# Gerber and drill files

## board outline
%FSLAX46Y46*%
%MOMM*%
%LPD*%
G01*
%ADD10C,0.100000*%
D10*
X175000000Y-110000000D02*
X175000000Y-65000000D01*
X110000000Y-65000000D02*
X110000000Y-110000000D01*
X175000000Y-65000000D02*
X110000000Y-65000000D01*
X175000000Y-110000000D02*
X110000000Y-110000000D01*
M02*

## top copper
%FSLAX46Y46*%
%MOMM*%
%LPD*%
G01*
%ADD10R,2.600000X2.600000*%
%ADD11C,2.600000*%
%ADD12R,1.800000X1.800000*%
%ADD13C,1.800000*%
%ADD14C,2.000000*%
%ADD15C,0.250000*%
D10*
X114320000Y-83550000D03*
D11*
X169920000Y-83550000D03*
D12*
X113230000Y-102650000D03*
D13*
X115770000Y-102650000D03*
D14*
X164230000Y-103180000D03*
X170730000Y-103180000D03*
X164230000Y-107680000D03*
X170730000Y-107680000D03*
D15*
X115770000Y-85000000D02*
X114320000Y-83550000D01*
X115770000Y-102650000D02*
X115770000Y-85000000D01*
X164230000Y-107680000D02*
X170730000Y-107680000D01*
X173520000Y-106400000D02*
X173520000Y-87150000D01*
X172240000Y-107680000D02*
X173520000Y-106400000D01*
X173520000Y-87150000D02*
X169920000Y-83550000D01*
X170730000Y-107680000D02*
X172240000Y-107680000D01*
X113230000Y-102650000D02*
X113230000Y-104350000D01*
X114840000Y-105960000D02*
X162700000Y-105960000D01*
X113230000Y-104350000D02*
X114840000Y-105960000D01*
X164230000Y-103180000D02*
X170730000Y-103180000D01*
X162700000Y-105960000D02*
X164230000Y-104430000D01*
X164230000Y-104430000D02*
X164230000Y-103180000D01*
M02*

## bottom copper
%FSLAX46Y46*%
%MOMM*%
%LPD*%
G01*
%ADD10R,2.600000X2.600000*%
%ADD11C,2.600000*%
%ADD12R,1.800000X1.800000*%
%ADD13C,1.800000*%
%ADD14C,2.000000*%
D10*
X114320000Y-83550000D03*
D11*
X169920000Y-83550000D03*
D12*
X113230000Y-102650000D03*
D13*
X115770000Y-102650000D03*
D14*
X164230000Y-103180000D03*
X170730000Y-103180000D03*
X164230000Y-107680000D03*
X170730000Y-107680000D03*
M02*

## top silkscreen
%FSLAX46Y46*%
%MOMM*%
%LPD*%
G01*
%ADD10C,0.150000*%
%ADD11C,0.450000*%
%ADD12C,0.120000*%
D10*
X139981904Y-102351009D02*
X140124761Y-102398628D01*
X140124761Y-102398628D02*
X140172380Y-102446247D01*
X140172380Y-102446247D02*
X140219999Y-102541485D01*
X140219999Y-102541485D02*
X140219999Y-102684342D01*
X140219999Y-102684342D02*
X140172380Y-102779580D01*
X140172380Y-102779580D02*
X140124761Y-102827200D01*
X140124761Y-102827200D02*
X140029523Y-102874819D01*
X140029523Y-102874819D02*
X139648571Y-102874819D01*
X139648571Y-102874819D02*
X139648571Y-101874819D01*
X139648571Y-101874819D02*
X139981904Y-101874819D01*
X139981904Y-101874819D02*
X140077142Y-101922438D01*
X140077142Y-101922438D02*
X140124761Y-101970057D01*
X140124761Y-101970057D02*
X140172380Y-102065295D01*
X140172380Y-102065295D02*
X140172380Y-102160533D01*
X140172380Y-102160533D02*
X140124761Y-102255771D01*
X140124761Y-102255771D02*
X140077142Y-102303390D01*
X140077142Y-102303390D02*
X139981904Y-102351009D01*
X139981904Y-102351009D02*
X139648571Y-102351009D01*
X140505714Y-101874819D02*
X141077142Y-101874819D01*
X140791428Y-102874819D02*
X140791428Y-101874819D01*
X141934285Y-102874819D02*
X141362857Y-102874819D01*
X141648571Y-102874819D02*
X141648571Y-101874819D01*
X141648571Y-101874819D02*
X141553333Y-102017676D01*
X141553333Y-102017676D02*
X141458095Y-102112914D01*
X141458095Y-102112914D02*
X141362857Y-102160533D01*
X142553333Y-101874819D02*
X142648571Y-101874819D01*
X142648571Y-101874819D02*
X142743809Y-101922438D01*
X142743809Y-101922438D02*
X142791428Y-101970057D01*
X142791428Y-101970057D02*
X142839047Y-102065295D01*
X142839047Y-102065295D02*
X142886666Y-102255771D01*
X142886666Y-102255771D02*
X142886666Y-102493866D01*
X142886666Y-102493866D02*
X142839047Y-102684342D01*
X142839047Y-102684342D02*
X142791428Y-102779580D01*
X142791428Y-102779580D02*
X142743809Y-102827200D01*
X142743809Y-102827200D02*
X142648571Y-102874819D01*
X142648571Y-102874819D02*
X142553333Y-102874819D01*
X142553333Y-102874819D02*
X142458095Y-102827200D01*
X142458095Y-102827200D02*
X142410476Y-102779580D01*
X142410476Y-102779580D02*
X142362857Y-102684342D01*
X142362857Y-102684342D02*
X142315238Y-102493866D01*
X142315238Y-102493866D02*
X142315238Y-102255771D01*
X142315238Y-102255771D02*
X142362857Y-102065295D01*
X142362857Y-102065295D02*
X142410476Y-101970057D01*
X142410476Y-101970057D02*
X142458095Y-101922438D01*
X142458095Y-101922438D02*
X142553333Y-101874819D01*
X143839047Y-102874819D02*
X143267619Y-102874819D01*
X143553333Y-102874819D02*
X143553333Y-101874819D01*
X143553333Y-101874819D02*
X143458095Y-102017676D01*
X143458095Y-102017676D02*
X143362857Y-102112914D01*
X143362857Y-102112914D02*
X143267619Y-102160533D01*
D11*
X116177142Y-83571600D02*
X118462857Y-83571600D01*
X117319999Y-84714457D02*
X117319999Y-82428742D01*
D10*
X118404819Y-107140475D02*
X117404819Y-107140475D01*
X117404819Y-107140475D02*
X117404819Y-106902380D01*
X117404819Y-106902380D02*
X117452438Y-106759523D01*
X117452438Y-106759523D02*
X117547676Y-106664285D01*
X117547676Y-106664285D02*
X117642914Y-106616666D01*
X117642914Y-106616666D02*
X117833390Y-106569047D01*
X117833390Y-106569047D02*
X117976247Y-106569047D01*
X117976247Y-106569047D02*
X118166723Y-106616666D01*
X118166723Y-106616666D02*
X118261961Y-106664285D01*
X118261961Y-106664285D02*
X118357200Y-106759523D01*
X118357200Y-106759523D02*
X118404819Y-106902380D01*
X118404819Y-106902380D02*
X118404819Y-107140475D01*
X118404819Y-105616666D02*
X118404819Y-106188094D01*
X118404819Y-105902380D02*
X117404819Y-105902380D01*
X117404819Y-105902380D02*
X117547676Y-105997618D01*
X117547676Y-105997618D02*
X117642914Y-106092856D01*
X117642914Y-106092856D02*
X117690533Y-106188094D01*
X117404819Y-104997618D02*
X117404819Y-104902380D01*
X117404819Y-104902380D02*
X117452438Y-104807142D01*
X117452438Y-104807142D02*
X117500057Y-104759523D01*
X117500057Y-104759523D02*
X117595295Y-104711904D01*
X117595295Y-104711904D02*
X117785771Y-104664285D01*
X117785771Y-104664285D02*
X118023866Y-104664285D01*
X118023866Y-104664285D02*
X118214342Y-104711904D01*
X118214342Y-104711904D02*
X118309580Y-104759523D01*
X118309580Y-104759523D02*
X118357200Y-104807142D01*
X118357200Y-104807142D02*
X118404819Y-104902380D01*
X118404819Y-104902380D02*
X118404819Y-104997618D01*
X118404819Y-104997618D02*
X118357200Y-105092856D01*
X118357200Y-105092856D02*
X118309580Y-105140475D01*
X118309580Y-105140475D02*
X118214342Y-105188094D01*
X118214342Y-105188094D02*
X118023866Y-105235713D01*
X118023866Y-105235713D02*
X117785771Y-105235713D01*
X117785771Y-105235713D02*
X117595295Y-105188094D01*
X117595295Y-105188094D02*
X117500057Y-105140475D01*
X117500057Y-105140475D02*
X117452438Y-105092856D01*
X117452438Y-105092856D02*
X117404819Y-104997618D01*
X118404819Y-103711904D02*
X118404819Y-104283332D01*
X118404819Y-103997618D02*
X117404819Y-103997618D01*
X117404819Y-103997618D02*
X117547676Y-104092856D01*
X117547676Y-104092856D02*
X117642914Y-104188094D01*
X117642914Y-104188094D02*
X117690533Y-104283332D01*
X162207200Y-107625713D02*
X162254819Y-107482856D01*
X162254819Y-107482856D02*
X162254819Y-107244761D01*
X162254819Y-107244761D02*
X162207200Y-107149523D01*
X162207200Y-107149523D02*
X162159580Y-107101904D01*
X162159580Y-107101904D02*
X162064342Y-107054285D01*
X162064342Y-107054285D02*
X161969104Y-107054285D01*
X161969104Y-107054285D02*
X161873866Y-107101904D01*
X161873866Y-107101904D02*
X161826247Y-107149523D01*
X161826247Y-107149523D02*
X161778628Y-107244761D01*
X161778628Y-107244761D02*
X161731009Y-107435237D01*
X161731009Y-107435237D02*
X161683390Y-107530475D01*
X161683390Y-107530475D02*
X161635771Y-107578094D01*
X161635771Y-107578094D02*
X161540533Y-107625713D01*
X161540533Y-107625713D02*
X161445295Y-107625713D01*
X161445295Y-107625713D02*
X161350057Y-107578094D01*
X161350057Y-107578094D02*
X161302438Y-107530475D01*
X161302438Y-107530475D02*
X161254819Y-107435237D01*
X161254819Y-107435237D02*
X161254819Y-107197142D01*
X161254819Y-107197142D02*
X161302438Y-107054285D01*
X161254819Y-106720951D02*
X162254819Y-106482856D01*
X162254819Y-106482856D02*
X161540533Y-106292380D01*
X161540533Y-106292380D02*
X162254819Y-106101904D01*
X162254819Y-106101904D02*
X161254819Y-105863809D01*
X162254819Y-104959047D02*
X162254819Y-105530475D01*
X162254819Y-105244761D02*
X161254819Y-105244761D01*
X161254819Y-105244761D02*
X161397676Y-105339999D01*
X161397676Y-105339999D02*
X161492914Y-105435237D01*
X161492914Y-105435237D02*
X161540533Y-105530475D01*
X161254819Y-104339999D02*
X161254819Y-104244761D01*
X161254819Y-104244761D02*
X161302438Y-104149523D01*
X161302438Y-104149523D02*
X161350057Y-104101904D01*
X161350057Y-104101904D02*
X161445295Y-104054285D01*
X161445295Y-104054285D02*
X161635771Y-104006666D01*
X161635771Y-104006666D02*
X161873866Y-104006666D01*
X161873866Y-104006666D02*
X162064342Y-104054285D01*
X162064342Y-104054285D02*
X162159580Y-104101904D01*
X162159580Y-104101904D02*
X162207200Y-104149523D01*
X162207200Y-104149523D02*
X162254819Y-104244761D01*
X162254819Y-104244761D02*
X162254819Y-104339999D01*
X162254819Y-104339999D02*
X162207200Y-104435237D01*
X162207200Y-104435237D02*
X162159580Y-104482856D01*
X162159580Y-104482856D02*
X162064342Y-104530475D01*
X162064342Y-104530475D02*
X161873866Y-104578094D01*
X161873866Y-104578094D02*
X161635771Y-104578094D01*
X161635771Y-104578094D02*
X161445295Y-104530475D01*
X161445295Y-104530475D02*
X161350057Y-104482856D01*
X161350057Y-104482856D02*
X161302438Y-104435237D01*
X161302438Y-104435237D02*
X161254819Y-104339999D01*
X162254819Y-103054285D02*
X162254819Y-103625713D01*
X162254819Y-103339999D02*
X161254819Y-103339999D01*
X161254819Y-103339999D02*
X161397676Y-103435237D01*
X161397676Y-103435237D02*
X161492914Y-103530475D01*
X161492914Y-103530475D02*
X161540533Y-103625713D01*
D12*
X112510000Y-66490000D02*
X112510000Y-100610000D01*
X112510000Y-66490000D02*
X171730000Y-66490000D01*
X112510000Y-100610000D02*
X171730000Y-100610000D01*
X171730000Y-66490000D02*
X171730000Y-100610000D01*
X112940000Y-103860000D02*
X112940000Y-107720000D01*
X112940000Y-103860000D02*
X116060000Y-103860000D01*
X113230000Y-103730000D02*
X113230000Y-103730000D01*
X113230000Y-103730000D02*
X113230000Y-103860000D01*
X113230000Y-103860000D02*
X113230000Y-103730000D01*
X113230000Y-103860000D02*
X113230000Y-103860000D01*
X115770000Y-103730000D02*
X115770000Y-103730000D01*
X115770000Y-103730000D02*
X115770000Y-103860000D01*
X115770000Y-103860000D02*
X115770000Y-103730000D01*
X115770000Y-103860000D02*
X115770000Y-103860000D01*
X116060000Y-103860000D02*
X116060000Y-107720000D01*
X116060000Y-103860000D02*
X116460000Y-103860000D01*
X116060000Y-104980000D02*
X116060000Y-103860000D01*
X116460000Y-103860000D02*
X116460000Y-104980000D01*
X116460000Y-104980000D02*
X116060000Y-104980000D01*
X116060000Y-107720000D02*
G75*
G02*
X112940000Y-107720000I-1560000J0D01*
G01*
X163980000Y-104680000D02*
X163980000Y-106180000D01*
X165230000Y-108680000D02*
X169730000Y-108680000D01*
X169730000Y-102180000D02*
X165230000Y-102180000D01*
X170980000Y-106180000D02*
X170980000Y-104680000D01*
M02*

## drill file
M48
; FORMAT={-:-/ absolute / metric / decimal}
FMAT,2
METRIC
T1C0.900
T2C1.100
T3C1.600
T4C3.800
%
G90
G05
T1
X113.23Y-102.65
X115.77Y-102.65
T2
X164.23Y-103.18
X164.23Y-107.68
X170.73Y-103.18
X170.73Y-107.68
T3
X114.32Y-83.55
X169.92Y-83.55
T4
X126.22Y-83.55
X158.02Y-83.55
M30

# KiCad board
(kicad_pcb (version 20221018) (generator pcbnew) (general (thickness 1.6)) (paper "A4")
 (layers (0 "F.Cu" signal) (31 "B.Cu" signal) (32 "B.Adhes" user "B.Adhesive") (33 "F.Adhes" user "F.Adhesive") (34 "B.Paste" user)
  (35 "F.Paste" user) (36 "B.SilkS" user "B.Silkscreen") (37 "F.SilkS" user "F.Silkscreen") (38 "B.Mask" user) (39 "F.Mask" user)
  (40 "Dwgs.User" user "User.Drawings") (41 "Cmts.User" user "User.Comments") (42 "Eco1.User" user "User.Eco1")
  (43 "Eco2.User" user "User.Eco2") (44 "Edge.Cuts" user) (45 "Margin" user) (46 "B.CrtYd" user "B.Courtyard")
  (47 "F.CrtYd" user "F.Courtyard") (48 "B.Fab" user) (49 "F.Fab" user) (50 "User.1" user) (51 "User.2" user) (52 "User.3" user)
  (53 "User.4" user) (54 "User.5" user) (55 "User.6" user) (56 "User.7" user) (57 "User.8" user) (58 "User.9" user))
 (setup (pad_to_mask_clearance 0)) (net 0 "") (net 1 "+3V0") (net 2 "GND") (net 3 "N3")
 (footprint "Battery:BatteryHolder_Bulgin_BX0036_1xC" (layer "F.Cu") (at 114.32 83.55)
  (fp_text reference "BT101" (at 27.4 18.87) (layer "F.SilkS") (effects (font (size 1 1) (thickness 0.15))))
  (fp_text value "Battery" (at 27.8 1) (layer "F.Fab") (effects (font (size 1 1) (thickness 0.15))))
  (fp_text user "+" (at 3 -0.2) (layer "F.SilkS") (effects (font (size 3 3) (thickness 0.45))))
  (fp_line (start -1.81 -17.06) (end -1.81 17.06) (stroke (width 0.12) (type solid)) (layer "F.SilkS"))
  (fp_line (start -1.81 -17.06) (end 57.41 -17.06) (stroke (width 0.12) (type solid)) (layer "F.SilkS"))
  (fp_line (start -1.81 17.06) (end 57.41 17.06) (stroke (width 0.12) (type solid)) (layer "F.SilkS"))
  (fp_line (start 57.41 -17.06) (end 57.41 17.06) (stroke (width 0.12) (type solid)) (layer "F.SilkS"))
  (pad "" np_thru_hole circle (at 11.9 0) (size 3.8 3.8) (drill 3.8) (layers "*.Cu" "*.Mask"))
  (pad "" np_thru_hole circle (at 43.7 0) (size 3.8 3.8) (drill 3.8) (layers "*.Cu" "*.Mask"))
  (pad "1" thru_hole rect (at 0 0) (size 2.6 2.6) (drill 1.6) (layers "*.Cu" "*.Mask") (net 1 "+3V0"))
  (pad "2" thru_hole circle (at 55.6 0) (size 2.6 2.6) (drill 1.6) (layers "*.Cu" "*.Mask") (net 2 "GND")))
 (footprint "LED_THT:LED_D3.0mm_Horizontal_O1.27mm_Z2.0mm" (layer "F.Cu") (at 113.23 102.65)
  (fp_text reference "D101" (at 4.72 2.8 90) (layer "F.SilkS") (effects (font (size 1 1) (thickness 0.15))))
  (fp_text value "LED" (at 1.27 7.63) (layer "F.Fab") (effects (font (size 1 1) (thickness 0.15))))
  (fp_line (start -0.29 1.21) (end -0.29 5.07) (stroke (width 0.12) (type solid)) (layer "F.SilkS"))
  (fp_line (start -0.29 1.21) (end 2.83 1.21) (stroke (width 0.12) (type solid)) (layer "F.SilkS"))
  (fp_line (start 0 1.08) (end 0 1.08) (stroke (width 0.12) (type solid)) (layer "F.SilkS"))
  (fp_line (start 0 1.08) (end 0 1.21) (stroke (width 0.12) (type solid)) (layer "F.SilkS"))
  (fp_line (start 0 1.21) (end 0 1.08) (stroke (width 0.12) (type solid)) (layer "F.SilkS"))
  (fp_line (start 0 1.21) (end 0 1.21) (stroke (width 0.12) (type solid)) (layer "F.SilkS"))
  (fp_line (start 2.54 1.08) (end 2.54 1.08) (stroke (width 0.12) (type solid)) (layer "F.SilkS"))
  (fp_line (start 2.54 1.08) (end 2.54 1.21) (stroke (width 0.12) (type solid)) (layer "F.SilkS"))
  (fp_line (start 2.54 1.21) (end 2.54 1.08) (stroke (width 0.12) (type solid)) (layer "F.SilkS"))
  (fp_line (start 2.54 1.21) (end 2.54 1.21) (stroke (width 0.12) (type solid)) (layer "F.SilkS"))
  (fp_line (start 2.83 1.21) (end 2.83 5.07) (stroke (width 0.12) (type solid)) (layer "F.SilkS"))
  (fp_line (start 2.83 1.21) (end 3.23 1.21) (stroke (width 0.12) (type solid)) (layer "F.SilkS"))
  (fp_line (start 2.83 2.33) (end 2.83 1.21) (stroke (width 0.12) (type solid)) (layer "F.SilkS"))
  (fp_line (start 3.23 1.21) (end 3.23 2.33) (stroke (width 0.12) (type solid)) (layer "F.SilkS"))
  (fp_line (start 3.23 2.33) (end 2.83 2.33) (stroke (width 0.12) (type solid)) (layer "F.SilkS"))
  (fp_arc (start 2.83 5.07) (mid 1.27 6.63) (end -0.29 5.07) (stroke (width 0.12) (type solid)) (layer "F.SilkS"))
  (pad "1" thru_hole rect (at 0 0) (size 1.8 1.8) (drill 0.9) (layers "*.Cu" "*.Mask") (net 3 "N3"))
  (pad "2" thru_hole circle (at 2.54 0) (size 1.8 1.8) (drill 0.9) (layers "*.Cu" "*.Mask") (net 1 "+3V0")))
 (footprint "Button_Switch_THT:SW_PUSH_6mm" (layer "F.Cu") (at 164.23 103.18)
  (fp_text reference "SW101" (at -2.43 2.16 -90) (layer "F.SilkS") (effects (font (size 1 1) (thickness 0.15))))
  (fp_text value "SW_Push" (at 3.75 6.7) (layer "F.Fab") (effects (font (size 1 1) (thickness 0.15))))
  (fp_line (start -0.25 1.5) (end -0.25 3) (stroke (width 0.12) (type solid)) (layer "F.SilkS"))
  (fp_line (start 1 5.5) (end 5.5 5.5) (stroke (width 0.12) (type solid)) (layer "F.SilkS"))
  (fp_line (start 5.5 -1) (end 1 -1) (stroke (width 0.12) (type solid)) (layer "F.SilkS"))
  (fp_line (start 6.75 3) (end 6.75 1.5) (stroke (width 0.12) (type solid)) (layer "F.SilkS"))
  (pad "1" thru_hole circle (at 0 0 90) (size 2 2) (drill 1.1) (layers "*.Cu" "*.Mask") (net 3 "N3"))
  (pad "1" thru_hole circle (at 6.5 0 90) (size 2 2) (drill 1.1) (layers "*.Cu" "*.Mask") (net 3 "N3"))
  (pad "2" thru_hole circle (at 0 4.5 90) (size 2 2) (drill 1.1) (layers "*.Cu" "*.Mask") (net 2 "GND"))
  (pad "2" thru_hole circle (at 6.5 4.5 90) (size 2 2) (drill 1.1) (layers "*.Cu" "*.Mask") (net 2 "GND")))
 (gr_line (start 175 110) (end 175 65) (stroke (width 0.1) (type default)) (layer "Edge.Cuts"))
 (gr_line (start 110 65) (end 110 110) (stroke (width 0.1) (type default)) (layer "Edge.Cuts"))
 (gr_line (start 175 65) (end 110 65) (stroke (width 0.1) (type default)) (layer "Edge.Cuts"))
 (gr_line (start 175 110) (end 110 110) (stroke (width 0.1) (type default)) (layer "Edge.Cuts"))
 (segment (start 115.77 85) (end 114.32 83.55) (width 0.25) (layer "F.Cu") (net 1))
 (segment (start 115.77 102.65) (end 115.77 85) (width 0.25) (layer "F.Cu") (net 1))
 (segment (start 164.23 107.68) (end 170.73 107.68) (width 0.25) (layer "F.Cu") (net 2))
 (segment (start 173.52 106.4) (end 173.52 87.15) (width 0.25) (layer "F.Cu") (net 2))
 (segment (start 172.24 107.68) (end 173.52 106.4) (width 0.25) (layer "F.Cu") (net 2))
 (segment (start 173.52 87.15) (end 169.92 83.55) (width 0.25) (layer "F.Cu") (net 2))
 (segment (start 170.73 107.68) (end 172.24 107.68) (width 0.25) (layer "F.Cu") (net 2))
 (segment (start 113.23 102.65) (end 113.23 104.35) (width 0.25) (layer "F.Cu") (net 3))
 (segment (start 114.84 105.96) (end 162.7 105.96) (width 0.25) (layer "F.Cu") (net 3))
 (segment (start 113.23 104.35) (end 114.84 105.96) (width 0.25) (layer "F.Cu") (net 3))
 (segment (start 164.23 103.18) (end 170.73 103.18) (width 0.25) (layer "F.Cu") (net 3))
 (segment (start 162.7 105.96) (end 164.23 104.43) (width 0.25) (layer "F.Cu") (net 3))
 (segment (start 164.23 104.43) (end 164.23 103.18) (width 0.25) (layer "F.Cu") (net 3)))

